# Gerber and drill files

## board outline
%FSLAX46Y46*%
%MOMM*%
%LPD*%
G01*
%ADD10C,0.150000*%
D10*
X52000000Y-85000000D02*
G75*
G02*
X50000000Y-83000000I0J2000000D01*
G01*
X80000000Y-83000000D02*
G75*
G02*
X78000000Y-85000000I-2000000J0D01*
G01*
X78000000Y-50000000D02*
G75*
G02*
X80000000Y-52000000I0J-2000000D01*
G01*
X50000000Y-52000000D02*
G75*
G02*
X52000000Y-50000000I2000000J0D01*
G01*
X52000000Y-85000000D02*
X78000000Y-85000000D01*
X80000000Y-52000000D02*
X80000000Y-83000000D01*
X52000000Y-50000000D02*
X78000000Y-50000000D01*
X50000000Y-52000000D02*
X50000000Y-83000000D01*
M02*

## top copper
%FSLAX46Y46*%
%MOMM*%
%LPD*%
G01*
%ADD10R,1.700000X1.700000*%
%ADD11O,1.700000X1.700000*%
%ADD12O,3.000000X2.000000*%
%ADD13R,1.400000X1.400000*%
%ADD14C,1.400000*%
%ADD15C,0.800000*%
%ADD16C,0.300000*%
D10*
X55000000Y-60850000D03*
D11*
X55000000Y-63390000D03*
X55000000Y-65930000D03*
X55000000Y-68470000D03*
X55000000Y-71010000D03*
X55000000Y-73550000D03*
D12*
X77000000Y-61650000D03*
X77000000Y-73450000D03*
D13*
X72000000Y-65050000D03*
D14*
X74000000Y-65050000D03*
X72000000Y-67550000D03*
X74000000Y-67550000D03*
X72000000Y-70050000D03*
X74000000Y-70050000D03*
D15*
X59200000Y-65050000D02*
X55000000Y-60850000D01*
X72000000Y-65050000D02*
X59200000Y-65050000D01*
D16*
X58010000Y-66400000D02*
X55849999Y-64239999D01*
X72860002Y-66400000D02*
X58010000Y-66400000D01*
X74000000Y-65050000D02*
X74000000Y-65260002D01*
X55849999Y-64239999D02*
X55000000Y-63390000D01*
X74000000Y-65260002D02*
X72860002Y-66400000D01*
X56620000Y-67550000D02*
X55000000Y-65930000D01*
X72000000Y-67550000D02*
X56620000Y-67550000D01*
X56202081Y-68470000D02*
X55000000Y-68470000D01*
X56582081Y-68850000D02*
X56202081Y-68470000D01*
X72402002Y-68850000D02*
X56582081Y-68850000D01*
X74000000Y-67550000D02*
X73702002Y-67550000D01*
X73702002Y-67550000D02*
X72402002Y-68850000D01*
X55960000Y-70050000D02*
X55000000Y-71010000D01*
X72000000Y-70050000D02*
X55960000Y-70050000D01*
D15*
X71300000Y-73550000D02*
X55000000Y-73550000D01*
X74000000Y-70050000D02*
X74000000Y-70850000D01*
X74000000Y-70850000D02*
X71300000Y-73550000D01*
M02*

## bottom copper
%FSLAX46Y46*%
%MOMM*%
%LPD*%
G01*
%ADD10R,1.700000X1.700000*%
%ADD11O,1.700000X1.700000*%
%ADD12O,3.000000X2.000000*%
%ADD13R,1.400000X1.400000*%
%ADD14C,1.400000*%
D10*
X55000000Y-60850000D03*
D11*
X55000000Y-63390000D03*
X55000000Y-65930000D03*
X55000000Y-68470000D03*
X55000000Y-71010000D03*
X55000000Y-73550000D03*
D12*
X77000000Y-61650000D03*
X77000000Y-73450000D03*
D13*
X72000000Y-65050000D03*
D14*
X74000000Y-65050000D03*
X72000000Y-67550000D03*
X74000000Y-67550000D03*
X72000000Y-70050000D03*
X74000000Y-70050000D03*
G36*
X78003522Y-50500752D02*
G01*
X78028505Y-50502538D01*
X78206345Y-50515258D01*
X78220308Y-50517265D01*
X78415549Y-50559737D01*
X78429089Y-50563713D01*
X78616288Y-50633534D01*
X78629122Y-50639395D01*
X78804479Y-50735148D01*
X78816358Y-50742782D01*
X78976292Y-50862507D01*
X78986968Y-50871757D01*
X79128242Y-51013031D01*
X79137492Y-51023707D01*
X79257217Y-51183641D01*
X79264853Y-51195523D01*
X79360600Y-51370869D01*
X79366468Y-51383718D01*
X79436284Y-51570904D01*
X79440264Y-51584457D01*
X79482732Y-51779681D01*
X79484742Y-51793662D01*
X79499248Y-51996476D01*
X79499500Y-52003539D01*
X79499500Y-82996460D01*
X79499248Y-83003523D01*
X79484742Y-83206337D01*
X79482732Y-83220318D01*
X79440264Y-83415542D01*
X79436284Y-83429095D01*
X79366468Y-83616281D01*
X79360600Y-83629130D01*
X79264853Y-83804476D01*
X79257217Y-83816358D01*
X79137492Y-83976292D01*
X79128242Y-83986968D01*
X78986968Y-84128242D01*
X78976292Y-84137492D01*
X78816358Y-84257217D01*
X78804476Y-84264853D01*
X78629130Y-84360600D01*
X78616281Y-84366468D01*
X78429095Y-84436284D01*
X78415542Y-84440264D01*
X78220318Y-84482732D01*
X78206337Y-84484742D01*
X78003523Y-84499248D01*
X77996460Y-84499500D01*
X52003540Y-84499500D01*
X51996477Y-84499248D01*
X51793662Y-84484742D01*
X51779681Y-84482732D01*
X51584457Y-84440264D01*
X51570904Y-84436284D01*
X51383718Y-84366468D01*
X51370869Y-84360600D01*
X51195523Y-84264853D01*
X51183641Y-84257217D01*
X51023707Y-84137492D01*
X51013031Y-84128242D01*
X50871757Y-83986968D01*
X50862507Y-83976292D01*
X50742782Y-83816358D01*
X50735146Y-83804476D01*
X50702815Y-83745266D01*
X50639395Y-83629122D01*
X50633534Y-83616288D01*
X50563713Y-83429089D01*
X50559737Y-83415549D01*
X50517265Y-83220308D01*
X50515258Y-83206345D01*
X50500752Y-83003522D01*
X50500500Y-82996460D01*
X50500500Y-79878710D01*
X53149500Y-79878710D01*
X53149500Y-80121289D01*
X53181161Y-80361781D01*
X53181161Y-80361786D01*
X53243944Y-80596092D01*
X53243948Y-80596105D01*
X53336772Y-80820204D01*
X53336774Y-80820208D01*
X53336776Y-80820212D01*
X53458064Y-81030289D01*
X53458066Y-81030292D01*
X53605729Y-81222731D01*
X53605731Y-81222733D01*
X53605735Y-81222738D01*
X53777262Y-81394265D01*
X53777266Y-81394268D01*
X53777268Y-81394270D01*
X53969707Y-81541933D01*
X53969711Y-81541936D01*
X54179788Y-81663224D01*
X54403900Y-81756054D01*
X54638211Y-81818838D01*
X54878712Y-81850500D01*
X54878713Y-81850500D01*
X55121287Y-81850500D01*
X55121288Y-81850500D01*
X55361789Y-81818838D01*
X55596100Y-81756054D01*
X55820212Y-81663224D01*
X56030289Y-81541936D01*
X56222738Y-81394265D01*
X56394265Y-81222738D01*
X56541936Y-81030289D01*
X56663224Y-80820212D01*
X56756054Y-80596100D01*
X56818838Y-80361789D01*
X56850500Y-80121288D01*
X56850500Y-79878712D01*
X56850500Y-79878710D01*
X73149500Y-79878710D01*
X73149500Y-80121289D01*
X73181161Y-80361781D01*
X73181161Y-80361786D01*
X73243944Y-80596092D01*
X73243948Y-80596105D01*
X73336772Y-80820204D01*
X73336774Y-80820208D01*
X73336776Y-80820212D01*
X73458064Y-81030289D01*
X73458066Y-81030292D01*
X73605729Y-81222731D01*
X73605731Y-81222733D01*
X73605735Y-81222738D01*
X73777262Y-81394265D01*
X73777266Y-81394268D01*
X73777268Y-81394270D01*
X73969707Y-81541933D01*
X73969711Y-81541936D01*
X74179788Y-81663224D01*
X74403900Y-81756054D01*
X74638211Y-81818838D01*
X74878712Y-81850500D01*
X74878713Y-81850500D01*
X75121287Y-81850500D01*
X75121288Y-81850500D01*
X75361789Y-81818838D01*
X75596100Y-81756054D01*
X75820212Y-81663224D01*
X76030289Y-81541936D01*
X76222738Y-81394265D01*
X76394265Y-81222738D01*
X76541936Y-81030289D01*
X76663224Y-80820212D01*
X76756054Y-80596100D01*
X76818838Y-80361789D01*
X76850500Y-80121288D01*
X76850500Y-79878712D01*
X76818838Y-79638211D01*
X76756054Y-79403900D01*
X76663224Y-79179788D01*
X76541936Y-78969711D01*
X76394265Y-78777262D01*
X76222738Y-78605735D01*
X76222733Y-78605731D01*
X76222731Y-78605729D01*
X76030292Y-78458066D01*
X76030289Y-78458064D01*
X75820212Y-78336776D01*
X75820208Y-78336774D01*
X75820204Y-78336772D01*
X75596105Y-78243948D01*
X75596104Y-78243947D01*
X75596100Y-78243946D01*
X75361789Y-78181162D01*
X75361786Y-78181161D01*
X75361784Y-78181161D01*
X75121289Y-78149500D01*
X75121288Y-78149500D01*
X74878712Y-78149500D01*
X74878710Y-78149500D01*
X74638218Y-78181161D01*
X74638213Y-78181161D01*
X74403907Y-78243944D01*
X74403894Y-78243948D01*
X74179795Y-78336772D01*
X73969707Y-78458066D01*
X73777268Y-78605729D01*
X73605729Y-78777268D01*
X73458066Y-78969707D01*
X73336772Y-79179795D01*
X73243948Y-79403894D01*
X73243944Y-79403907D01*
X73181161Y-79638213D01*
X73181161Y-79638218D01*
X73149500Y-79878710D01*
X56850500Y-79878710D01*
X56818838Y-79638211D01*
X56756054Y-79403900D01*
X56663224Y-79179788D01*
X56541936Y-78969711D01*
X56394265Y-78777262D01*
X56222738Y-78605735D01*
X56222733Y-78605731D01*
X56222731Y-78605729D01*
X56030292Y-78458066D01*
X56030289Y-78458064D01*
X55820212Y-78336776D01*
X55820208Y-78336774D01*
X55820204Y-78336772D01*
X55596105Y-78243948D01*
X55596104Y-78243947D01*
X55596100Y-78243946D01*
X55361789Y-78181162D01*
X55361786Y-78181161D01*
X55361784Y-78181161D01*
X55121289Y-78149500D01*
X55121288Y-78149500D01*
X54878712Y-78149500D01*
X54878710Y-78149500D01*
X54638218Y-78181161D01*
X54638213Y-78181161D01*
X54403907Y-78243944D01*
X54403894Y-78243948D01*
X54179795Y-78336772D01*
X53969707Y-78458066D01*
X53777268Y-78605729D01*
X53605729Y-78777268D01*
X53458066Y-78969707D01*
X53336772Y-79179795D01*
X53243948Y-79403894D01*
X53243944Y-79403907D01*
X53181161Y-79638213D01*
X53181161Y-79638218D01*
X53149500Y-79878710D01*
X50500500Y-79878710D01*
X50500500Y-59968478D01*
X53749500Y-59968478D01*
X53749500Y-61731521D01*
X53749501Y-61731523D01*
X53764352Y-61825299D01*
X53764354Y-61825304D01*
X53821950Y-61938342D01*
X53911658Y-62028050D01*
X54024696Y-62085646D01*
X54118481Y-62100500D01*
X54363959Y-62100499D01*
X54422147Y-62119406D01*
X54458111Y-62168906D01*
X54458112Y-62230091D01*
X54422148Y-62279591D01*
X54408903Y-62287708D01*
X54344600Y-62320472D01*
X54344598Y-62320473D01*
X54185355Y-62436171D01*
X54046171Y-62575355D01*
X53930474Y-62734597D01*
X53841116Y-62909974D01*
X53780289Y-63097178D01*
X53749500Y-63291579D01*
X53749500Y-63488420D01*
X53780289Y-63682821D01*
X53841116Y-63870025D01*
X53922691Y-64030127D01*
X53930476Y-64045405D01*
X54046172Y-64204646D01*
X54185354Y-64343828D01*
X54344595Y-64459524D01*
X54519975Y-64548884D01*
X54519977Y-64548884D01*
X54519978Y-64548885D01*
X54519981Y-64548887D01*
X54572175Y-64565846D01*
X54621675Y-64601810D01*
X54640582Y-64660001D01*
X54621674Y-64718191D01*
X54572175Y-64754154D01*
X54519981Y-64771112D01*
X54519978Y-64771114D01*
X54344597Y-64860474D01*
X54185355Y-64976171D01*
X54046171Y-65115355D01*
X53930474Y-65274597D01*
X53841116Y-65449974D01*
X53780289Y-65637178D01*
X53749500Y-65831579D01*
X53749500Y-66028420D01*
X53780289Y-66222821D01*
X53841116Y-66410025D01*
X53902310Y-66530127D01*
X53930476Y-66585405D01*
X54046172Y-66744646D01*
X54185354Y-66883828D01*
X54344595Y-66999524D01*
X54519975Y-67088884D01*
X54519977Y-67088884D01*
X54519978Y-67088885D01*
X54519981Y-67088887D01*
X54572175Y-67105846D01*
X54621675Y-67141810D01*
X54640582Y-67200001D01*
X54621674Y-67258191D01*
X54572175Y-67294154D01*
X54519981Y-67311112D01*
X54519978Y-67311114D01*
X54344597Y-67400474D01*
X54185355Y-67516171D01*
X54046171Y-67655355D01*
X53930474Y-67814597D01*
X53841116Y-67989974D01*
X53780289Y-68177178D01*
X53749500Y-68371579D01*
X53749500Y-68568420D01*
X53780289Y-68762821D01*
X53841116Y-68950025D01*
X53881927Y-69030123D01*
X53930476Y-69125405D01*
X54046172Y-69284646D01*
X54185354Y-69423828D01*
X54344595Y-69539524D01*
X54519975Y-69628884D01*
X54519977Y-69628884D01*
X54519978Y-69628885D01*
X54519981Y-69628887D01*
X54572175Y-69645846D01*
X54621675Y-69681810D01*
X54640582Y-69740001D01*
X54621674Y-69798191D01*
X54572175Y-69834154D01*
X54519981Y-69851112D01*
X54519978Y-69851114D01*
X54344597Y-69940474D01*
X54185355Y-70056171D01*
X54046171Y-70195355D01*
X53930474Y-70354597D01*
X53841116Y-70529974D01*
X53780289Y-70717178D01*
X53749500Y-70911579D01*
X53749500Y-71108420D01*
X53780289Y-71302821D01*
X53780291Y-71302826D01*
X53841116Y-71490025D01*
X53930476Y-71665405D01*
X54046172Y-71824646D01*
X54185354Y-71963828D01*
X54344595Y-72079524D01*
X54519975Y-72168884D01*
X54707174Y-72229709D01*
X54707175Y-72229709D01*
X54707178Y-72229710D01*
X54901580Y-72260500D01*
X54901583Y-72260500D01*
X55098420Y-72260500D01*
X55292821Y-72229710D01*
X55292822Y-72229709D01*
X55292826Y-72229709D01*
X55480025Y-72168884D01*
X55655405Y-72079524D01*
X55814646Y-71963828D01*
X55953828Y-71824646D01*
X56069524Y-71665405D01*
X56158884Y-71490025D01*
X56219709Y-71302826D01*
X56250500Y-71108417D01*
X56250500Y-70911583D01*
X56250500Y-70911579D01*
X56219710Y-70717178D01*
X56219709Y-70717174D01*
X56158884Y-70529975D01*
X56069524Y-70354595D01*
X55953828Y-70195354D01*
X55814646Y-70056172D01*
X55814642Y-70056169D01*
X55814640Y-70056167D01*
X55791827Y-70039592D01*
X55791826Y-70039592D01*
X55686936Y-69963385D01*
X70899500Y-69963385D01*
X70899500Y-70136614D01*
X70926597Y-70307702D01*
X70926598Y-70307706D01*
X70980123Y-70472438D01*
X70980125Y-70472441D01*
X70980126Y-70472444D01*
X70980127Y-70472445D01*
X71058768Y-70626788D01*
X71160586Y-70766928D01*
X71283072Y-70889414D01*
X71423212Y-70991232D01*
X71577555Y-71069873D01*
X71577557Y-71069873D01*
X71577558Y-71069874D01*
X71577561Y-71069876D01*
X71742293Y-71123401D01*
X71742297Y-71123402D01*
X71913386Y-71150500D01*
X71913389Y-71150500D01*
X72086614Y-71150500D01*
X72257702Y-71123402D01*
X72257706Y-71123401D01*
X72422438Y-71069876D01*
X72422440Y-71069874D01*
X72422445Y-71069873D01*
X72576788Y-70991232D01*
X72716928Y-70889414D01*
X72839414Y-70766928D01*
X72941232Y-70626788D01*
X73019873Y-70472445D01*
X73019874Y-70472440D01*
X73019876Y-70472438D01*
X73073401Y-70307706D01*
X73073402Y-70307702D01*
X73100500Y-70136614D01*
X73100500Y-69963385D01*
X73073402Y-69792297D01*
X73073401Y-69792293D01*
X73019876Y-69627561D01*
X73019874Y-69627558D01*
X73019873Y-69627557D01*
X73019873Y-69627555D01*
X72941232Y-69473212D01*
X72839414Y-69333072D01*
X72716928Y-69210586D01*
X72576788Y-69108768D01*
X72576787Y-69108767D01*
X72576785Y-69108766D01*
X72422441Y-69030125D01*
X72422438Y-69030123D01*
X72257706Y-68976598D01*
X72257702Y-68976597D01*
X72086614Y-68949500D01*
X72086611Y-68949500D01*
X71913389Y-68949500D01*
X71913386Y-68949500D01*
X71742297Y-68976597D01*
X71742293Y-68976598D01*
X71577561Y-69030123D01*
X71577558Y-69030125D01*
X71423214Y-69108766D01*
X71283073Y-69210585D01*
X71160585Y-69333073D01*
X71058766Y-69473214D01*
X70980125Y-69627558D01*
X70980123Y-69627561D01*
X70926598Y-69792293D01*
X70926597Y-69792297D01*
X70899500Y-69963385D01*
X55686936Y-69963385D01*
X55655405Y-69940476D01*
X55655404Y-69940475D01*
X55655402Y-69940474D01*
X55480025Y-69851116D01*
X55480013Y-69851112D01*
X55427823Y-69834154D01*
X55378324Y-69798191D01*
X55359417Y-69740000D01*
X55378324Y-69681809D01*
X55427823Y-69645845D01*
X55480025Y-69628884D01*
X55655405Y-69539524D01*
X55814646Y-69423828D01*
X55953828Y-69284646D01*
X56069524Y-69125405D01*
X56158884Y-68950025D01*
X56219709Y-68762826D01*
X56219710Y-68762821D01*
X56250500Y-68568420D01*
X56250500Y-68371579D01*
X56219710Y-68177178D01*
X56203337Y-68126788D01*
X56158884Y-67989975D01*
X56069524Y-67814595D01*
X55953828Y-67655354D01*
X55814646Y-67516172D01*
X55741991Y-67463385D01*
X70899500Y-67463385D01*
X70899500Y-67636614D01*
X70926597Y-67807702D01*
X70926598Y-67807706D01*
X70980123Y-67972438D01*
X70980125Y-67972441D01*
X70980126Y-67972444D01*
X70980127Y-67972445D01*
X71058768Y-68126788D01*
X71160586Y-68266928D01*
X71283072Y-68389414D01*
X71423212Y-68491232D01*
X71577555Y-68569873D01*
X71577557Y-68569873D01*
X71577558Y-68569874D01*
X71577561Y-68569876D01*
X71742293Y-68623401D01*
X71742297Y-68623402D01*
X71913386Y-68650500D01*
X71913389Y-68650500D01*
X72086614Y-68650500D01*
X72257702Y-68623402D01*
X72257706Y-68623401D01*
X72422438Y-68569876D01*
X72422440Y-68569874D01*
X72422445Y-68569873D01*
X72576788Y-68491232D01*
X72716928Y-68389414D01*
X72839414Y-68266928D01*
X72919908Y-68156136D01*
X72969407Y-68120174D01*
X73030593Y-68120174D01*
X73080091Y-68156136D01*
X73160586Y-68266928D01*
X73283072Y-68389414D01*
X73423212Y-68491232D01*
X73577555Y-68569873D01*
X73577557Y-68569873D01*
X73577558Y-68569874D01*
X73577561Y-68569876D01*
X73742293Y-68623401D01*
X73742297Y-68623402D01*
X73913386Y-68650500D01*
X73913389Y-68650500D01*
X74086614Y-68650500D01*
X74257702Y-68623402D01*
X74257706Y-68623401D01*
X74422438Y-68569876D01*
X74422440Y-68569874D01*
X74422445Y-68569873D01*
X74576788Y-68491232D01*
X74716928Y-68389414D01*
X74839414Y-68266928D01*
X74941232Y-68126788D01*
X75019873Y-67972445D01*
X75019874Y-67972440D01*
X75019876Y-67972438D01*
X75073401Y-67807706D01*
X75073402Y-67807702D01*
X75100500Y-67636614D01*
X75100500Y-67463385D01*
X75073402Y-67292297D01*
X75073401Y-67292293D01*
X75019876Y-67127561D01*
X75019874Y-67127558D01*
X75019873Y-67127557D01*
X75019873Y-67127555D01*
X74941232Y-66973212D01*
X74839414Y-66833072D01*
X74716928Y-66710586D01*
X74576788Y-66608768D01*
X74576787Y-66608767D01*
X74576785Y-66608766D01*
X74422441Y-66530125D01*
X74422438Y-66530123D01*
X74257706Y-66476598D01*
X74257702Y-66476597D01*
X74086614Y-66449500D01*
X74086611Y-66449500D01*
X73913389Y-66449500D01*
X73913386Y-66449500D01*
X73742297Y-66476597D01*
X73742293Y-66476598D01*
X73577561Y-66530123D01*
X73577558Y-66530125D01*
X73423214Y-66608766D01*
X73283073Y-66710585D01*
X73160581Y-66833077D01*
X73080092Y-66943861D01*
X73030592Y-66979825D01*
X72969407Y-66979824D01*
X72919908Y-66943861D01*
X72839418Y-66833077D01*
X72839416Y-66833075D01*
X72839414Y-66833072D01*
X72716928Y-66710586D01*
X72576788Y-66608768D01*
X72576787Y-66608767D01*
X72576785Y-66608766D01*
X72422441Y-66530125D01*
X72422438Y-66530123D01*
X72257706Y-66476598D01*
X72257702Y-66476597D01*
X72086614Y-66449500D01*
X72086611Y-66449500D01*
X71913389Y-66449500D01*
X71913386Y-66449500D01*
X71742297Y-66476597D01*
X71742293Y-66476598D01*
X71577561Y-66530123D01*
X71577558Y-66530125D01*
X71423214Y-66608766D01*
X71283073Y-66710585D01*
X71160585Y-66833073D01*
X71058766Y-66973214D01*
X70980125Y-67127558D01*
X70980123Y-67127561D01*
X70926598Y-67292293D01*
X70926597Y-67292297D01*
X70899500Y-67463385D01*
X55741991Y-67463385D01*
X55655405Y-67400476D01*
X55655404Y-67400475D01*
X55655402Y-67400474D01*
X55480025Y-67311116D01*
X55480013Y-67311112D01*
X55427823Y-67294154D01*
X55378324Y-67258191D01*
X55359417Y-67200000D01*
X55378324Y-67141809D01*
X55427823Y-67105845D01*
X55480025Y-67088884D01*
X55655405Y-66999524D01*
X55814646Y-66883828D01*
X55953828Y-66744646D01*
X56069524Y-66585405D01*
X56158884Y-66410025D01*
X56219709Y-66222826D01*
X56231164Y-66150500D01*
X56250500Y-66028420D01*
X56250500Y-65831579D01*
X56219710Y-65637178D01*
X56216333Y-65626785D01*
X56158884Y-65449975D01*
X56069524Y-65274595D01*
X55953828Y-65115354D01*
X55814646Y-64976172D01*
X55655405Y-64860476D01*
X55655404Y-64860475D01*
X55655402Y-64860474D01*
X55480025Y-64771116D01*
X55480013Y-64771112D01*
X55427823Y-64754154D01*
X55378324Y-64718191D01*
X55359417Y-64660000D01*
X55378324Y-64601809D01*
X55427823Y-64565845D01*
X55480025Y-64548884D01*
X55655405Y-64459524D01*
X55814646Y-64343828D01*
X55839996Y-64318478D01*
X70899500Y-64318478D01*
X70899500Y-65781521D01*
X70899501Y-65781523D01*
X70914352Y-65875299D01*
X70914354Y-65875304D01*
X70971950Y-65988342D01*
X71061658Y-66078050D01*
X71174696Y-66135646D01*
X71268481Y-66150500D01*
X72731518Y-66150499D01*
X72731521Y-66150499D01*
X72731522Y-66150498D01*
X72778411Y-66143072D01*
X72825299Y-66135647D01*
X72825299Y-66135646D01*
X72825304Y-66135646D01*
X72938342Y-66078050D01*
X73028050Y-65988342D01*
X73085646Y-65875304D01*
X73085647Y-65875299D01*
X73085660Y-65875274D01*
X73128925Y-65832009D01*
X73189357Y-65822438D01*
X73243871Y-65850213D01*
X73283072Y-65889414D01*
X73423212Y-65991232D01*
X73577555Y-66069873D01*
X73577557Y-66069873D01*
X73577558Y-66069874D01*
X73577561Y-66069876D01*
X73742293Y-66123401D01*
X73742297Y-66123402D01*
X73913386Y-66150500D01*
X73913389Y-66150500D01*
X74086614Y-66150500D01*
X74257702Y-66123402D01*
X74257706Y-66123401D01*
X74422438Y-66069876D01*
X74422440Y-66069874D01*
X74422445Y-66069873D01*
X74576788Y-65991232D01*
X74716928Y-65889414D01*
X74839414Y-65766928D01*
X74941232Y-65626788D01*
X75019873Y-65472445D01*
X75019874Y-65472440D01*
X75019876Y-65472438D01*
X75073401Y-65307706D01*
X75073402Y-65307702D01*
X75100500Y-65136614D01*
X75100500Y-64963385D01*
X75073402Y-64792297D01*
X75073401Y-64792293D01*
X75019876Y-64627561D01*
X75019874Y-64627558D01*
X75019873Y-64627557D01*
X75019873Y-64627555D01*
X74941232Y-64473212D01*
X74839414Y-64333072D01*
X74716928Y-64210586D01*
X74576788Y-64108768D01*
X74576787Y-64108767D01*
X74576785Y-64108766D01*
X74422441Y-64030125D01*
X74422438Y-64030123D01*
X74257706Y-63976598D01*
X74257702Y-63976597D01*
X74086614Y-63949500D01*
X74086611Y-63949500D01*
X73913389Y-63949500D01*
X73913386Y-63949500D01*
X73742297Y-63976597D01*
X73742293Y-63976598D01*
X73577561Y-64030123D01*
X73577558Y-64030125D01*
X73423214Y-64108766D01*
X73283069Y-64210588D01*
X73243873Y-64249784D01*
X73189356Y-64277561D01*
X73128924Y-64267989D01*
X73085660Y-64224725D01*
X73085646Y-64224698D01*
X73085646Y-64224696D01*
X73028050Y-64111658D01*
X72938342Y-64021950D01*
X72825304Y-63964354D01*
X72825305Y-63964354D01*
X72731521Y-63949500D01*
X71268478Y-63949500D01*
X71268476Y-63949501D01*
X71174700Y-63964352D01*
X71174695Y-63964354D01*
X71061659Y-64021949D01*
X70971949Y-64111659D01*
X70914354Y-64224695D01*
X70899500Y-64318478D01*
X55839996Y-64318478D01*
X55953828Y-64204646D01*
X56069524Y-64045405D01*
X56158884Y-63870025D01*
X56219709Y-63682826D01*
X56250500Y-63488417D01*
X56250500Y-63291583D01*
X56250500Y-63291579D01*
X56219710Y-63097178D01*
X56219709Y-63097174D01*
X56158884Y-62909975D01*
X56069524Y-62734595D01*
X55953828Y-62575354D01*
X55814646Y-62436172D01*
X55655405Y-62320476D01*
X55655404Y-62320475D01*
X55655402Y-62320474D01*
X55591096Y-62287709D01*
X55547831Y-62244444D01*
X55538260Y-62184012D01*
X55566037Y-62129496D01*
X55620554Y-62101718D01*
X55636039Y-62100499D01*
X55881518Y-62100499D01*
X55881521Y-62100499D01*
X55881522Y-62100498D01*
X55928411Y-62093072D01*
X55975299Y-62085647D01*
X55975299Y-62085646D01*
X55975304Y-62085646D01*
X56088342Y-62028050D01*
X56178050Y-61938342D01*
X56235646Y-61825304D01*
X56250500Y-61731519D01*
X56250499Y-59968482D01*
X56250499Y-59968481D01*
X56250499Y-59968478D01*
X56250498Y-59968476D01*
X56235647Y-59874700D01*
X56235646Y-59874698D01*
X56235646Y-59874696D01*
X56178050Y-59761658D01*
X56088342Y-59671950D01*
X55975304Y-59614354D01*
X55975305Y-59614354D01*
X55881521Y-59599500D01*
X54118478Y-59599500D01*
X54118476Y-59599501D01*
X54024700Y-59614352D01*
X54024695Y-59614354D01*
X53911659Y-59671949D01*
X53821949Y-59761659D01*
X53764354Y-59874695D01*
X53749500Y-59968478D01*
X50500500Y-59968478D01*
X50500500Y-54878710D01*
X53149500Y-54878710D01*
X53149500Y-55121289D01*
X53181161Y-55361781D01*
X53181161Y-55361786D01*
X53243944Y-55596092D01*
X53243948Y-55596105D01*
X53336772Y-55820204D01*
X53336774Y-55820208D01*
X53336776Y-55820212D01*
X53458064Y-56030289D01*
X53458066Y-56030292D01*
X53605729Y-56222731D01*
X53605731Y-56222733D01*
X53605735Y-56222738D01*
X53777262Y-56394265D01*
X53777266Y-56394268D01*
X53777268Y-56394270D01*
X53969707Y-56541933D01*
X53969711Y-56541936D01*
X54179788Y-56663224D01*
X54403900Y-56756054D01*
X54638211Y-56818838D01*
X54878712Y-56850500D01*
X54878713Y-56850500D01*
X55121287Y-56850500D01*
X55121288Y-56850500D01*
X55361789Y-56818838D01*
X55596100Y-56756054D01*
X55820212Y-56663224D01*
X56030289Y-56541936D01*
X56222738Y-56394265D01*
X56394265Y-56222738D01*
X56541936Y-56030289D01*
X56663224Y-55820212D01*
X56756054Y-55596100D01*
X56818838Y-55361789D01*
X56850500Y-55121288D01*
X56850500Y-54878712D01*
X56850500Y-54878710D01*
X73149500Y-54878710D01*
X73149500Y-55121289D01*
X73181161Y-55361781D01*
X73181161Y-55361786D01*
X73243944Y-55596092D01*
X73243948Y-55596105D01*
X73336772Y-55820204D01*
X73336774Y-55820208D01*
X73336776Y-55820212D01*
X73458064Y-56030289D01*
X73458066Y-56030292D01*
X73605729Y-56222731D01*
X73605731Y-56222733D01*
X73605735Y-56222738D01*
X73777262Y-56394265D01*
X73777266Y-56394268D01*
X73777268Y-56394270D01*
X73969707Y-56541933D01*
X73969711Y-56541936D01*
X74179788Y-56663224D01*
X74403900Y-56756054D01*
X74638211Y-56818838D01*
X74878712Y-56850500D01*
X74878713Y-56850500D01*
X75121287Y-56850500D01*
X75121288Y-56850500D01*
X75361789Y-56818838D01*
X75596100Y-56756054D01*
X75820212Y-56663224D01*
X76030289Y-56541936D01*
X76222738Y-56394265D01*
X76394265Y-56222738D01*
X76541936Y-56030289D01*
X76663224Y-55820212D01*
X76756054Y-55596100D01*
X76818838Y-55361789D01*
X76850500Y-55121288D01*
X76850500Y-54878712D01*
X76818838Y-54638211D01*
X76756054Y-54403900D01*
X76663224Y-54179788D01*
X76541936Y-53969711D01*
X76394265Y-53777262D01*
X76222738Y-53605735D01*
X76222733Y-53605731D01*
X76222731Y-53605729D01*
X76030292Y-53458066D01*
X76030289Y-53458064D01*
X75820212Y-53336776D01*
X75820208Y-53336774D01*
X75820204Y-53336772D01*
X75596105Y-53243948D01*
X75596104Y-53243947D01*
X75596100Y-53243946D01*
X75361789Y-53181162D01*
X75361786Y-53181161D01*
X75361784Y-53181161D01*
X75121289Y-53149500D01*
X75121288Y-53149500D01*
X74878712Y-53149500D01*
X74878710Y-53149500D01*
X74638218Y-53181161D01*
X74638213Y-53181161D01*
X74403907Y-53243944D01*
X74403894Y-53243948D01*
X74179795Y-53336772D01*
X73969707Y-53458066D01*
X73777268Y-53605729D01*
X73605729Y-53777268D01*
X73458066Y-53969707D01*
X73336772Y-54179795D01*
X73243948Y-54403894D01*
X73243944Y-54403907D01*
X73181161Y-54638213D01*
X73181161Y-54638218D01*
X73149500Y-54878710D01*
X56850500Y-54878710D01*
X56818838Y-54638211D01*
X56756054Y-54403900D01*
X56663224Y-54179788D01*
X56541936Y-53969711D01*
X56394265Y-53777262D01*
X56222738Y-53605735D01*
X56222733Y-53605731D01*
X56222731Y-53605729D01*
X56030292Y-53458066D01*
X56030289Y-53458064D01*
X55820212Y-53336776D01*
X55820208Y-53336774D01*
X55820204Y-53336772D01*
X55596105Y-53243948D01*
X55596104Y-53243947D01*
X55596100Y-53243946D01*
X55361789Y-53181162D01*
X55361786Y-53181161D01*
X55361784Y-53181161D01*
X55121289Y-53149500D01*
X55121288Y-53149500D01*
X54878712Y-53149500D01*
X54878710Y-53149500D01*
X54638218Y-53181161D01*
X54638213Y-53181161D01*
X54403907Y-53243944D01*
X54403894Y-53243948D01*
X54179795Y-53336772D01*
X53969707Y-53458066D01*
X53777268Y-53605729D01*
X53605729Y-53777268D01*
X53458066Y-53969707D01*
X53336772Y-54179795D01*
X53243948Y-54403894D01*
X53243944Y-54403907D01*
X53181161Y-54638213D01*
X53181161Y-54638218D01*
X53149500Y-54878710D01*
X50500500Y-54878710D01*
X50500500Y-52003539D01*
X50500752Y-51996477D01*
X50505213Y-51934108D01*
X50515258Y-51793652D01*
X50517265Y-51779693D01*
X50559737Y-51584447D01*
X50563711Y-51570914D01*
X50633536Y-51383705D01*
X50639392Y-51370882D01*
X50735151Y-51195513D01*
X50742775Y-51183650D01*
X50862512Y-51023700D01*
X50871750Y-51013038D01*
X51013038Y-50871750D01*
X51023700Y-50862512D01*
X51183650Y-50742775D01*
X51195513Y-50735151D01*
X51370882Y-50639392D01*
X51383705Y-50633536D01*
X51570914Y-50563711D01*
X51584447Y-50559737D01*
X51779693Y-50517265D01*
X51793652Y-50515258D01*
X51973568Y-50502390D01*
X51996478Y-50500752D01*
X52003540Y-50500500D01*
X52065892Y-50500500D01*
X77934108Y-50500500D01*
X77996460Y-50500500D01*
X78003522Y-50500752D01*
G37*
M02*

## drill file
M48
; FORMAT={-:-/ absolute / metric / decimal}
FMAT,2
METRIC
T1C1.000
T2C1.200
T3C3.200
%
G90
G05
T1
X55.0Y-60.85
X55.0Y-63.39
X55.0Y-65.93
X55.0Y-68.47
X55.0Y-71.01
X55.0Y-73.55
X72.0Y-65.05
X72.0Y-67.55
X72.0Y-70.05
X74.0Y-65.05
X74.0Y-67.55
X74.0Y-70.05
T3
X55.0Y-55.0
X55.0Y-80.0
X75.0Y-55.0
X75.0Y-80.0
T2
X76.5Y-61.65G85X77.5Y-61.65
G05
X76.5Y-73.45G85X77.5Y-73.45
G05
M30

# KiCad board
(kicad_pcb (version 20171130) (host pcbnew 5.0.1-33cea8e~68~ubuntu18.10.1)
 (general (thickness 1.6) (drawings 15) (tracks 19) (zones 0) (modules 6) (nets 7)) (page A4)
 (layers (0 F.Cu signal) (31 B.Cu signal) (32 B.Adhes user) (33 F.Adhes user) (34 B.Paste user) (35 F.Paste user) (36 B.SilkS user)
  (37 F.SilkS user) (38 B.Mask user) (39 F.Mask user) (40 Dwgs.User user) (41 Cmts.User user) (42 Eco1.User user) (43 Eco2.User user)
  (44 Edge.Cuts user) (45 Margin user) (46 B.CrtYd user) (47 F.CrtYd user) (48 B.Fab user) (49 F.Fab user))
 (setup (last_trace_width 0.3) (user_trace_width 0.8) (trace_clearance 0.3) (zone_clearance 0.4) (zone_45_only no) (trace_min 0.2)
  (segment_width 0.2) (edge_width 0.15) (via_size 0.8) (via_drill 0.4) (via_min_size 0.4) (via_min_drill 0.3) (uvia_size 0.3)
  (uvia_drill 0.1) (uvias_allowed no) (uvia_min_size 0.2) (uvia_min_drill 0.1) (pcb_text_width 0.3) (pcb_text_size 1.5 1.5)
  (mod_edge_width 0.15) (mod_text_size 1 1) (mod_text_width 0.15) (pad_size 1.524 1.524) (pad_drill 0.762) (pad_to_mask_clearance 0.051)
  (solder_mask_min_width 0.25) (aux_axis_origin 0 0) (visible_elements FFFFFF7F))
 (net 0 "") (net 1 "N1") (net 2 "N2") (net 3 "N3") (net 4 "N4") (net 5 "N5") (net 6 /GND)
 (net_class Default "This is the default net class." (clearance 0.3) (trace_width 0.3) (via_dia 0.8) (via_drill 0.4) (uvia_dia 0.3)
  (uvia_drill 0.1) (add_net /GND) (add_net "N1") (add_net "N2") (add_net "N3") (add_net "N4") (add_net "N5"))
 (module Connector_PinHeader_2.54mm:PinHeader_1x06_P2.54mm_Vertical (layer F.Cu) (at 55 60.85)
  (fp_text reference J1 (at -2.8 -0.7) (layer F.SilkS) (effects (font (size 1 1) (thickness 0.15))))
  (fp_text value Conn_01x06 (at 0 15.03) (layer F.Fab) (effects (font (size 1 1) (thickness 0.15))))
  (pad 1 thru_hole rect (at 0 0) (size 1.7 1.7) (drill 1) (layers *.Cu *.Mask) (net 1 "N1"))
  (pad 2 thru_hole oval (at 0 2.54) (size 1.7 1.7) (drill 1) (layers *.Cu *.Mask) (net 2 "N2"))
  (pad 3 thru_hole oval (at 0 5.08) (size 1.7 1.7) (drill 1) (layers *.Cu *.Mask) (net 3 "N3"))
  (pad 4 thru_hole oval (at 0 7.62) (size 1.7 1.7) (drill 1) (layers *.Cu *.Mask) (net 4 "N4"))
  (pad 5 thru_hole oval (at 0 10.16) (size 1.7 1.7) (drill 1) (layers *.Cu *.Mask) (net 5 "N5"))
  (pad 6 thru_hole oval (at 0 12.7) (size 1.7 1.7) (drill 1) (layers *.Cu *.Mask) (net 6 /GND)))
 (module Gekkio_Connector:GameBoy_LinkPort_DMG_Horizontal (layer F.Cu) (at 72 65.05)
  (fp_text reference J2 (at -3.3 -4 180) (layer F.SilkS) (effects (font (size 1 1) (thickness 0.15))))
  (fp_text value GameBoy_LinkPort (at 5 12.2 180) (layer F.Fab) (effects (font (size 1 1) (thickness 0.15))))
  (pad SH thru_hole oval (at 5 -3.4 90) (size 2 3) (drill oval 1.2 2.2) (layers *.Cu *.Mask) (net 6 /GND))
  (pad SH thru_hole oval (at 5 8.4 90) (size 2 3) (drill oval 1.2 2.2) (layers *.Cu *.Mask) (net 6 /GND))
  (pad 1 thru_hole rect (at 0 0 90) (size 1.4 1.4) (drill 1) (layers *.Cu *.Mask) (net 1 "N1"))
  (pad 2 thru_hole circle (at 2 0 90) (size 1.4 1.4) (drill 1) (layers *.Cu *.Mask) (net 2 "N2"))
  (pad 3 thru_hole circle (at 0 2.5 90) (size 1.4 1.4) (drill 1) (layers *.Cu *.Mask) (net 3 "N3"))
  (pad 4 thru_hole circle (at 2 2.5 90) (size 1.4 1.4) (drill 1) (layers *.Cu *.Mask) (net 4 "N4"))
  (pad 5 thru_hole circle (at 0 5 90) (size 1.4 1.4) (drill 1) (layers *.Cu *.Mask) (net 5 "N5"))
  (pad 6 thru_hole circle (at 2 5 90) (size 1.4 1.4) (drill 1) (layers *.Cu *.Mask) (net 6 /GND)))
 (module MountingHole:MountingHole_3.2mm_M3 (layer F.Cu) (at 75 80)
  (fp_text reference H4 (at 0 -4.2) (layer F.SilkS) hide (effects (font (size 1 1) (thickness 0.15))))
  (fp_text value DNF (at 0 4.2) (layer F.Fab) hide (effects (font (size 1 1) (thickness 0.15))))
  (pad 1 np_thru_hole circle (at 0 0) (size 3.2 3.2) (drill 3.2) (layers *.Cu *.Mask)))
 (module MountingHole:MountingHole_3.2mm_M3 (layer F.Cu) (at 75 55)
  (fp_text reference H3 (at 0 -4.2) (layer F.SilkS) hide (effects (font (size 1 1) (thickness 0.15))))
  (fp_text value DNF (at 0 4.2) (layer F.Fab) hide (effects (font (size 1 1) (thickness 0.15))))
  (pad 1 np_thru_hole circle (at 0 0) (size 3.2 3.2) (drill 3.2) (layers *.Cu *.Mask)))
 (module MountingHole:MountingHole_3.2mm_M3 (layer F.Cu) (at 55 80)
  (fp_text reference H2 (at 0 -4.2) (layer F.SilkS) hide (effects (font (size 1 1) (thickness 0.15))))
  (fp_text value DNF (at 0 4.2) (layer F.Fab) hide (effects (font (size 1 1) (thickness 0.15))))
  (pad 1 np_thru_hole circle (at 0 0) (size 3.2 3.2) (drill 3.2) (layers *.Cu *.Mask)))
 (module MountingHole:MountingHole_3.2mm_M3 (layer F.Cu) (at 55 55)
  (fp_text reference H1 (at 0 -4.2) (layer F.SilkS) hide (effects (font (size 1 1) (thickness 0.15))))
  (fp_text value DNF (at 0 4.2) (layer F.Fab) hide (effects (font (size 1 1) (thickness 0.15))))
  (pad 1 np_thru_hole circle (at 0 0) (size 3.2 3.2) (drill 3.2) (layers *.Cu *.Mask)))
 (gr_arc (start 52 83) (end 50 83) (angle -90) (layer Edge.Cuts) (width 0.15))
 (gr_arc (start 78 83) (end 78 85) (angle -90) (layer Edge.Cuts) (width 0.15))
 (gr_arc (start 78 52) (end 80 52) (angle -90) (layer Edge.Cuts) (width 0.15))
 (gr_arc (start 52 52) (end 52 50) (angle -90) (layer Edge.Cuts) (width 0.15))
 (gr_line (start 52 85) (end 78 85) (layer Edge.Cuts) (width 0.15))
 (gr_line (start 80 52) (end 80 83) (layer Edge.Cuts) (width 0.15))
 (gr_line (start 52 50) (end 78 50) (layer Edge.Cuts) (width 0.15))
 (gr_line (start 50 52) (end 50 83) (layer Edge.Cuts) (width 0.15))
 (segment (start 59.2 65.05) (end 55 60.85) (width 0.8) (layer F.Cu) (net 1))
 (segment (start 72 65.05) (end 59.2 65.05) (width 0.8) (layer F.Cu) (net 1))
 (segment (start 58.01 66.4) (end 55.849999 64.239999) (width 0.3) (layer F.Cu) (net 2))
 (segment (start 72.860002 66.4) (end 58.01 66.4) (width 0.3) (layer F.Cu) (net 2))
 (segment (start 74 65.05) (end 74 65.260002) (width 0.3) (layer F.Cu) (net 2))
 (segment (start 55.849999 64.239999) (end 55 63.39) (width 0.3) (layer F.Cu) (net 2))
 (segment (start 74 65.260002) (end 72.860002 66.4) (width 0.3) (layer F.Cu) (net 2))
 (segment (start 56.62 67.55) (end 55 65.93) (width 0.3) (layer F.Cu) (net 3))
 (segment (start 72 67.55) (end 56.62 67.55) (width 0.3) (layer F.Cu) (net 3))
 (segment (start 56.202081 68.47) (end 55 68.47) (width 0.3) (layer F.Cu) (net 4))
 (segment (start 56.582081 68.85) (end 56.202081 68.47) (width 0.3) (layer F.Cu) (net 4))
 (segment (start 72.402002 68.85) (end 56.582081 68.85) (width 0.3) (layer F.Cu) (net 4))
 (segment (start 74 67.55) (end 73.702002 67.55) (width 0.3) (layer F.Cu) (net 4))
 (segment (start 73.702002 67.55) (end 72.402002 68.85) (width 0.3) (layer F.Cu) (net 4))
 (segment (start 55.96 70.05) (end 55 71.01) (width 0.3) (layer F.Cu) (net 5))
 (segment (start 72 70.05) (end 55.96 70.05) (width 0.3) (layer F.Cu) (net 5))
 (segment (start 71.3 73.55) (end 55 73.55) (width 0.8) (layer F.Cu) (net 6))
 (segment (start 74 70.05) (end 74 70.85) (width 0.8) (layer F.Cu) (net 6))
 (segment (start 74 70.85) (end 71.3 73.55) (width 0.8) (layer F.Cu) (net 6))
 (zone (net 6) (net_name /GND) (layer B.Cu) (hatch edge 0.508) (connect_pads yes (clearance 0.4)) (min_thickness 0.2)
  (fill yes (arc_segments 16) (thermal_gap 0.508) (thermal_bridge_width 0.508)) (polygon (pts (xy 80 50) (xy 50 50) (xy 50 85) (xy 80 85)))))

